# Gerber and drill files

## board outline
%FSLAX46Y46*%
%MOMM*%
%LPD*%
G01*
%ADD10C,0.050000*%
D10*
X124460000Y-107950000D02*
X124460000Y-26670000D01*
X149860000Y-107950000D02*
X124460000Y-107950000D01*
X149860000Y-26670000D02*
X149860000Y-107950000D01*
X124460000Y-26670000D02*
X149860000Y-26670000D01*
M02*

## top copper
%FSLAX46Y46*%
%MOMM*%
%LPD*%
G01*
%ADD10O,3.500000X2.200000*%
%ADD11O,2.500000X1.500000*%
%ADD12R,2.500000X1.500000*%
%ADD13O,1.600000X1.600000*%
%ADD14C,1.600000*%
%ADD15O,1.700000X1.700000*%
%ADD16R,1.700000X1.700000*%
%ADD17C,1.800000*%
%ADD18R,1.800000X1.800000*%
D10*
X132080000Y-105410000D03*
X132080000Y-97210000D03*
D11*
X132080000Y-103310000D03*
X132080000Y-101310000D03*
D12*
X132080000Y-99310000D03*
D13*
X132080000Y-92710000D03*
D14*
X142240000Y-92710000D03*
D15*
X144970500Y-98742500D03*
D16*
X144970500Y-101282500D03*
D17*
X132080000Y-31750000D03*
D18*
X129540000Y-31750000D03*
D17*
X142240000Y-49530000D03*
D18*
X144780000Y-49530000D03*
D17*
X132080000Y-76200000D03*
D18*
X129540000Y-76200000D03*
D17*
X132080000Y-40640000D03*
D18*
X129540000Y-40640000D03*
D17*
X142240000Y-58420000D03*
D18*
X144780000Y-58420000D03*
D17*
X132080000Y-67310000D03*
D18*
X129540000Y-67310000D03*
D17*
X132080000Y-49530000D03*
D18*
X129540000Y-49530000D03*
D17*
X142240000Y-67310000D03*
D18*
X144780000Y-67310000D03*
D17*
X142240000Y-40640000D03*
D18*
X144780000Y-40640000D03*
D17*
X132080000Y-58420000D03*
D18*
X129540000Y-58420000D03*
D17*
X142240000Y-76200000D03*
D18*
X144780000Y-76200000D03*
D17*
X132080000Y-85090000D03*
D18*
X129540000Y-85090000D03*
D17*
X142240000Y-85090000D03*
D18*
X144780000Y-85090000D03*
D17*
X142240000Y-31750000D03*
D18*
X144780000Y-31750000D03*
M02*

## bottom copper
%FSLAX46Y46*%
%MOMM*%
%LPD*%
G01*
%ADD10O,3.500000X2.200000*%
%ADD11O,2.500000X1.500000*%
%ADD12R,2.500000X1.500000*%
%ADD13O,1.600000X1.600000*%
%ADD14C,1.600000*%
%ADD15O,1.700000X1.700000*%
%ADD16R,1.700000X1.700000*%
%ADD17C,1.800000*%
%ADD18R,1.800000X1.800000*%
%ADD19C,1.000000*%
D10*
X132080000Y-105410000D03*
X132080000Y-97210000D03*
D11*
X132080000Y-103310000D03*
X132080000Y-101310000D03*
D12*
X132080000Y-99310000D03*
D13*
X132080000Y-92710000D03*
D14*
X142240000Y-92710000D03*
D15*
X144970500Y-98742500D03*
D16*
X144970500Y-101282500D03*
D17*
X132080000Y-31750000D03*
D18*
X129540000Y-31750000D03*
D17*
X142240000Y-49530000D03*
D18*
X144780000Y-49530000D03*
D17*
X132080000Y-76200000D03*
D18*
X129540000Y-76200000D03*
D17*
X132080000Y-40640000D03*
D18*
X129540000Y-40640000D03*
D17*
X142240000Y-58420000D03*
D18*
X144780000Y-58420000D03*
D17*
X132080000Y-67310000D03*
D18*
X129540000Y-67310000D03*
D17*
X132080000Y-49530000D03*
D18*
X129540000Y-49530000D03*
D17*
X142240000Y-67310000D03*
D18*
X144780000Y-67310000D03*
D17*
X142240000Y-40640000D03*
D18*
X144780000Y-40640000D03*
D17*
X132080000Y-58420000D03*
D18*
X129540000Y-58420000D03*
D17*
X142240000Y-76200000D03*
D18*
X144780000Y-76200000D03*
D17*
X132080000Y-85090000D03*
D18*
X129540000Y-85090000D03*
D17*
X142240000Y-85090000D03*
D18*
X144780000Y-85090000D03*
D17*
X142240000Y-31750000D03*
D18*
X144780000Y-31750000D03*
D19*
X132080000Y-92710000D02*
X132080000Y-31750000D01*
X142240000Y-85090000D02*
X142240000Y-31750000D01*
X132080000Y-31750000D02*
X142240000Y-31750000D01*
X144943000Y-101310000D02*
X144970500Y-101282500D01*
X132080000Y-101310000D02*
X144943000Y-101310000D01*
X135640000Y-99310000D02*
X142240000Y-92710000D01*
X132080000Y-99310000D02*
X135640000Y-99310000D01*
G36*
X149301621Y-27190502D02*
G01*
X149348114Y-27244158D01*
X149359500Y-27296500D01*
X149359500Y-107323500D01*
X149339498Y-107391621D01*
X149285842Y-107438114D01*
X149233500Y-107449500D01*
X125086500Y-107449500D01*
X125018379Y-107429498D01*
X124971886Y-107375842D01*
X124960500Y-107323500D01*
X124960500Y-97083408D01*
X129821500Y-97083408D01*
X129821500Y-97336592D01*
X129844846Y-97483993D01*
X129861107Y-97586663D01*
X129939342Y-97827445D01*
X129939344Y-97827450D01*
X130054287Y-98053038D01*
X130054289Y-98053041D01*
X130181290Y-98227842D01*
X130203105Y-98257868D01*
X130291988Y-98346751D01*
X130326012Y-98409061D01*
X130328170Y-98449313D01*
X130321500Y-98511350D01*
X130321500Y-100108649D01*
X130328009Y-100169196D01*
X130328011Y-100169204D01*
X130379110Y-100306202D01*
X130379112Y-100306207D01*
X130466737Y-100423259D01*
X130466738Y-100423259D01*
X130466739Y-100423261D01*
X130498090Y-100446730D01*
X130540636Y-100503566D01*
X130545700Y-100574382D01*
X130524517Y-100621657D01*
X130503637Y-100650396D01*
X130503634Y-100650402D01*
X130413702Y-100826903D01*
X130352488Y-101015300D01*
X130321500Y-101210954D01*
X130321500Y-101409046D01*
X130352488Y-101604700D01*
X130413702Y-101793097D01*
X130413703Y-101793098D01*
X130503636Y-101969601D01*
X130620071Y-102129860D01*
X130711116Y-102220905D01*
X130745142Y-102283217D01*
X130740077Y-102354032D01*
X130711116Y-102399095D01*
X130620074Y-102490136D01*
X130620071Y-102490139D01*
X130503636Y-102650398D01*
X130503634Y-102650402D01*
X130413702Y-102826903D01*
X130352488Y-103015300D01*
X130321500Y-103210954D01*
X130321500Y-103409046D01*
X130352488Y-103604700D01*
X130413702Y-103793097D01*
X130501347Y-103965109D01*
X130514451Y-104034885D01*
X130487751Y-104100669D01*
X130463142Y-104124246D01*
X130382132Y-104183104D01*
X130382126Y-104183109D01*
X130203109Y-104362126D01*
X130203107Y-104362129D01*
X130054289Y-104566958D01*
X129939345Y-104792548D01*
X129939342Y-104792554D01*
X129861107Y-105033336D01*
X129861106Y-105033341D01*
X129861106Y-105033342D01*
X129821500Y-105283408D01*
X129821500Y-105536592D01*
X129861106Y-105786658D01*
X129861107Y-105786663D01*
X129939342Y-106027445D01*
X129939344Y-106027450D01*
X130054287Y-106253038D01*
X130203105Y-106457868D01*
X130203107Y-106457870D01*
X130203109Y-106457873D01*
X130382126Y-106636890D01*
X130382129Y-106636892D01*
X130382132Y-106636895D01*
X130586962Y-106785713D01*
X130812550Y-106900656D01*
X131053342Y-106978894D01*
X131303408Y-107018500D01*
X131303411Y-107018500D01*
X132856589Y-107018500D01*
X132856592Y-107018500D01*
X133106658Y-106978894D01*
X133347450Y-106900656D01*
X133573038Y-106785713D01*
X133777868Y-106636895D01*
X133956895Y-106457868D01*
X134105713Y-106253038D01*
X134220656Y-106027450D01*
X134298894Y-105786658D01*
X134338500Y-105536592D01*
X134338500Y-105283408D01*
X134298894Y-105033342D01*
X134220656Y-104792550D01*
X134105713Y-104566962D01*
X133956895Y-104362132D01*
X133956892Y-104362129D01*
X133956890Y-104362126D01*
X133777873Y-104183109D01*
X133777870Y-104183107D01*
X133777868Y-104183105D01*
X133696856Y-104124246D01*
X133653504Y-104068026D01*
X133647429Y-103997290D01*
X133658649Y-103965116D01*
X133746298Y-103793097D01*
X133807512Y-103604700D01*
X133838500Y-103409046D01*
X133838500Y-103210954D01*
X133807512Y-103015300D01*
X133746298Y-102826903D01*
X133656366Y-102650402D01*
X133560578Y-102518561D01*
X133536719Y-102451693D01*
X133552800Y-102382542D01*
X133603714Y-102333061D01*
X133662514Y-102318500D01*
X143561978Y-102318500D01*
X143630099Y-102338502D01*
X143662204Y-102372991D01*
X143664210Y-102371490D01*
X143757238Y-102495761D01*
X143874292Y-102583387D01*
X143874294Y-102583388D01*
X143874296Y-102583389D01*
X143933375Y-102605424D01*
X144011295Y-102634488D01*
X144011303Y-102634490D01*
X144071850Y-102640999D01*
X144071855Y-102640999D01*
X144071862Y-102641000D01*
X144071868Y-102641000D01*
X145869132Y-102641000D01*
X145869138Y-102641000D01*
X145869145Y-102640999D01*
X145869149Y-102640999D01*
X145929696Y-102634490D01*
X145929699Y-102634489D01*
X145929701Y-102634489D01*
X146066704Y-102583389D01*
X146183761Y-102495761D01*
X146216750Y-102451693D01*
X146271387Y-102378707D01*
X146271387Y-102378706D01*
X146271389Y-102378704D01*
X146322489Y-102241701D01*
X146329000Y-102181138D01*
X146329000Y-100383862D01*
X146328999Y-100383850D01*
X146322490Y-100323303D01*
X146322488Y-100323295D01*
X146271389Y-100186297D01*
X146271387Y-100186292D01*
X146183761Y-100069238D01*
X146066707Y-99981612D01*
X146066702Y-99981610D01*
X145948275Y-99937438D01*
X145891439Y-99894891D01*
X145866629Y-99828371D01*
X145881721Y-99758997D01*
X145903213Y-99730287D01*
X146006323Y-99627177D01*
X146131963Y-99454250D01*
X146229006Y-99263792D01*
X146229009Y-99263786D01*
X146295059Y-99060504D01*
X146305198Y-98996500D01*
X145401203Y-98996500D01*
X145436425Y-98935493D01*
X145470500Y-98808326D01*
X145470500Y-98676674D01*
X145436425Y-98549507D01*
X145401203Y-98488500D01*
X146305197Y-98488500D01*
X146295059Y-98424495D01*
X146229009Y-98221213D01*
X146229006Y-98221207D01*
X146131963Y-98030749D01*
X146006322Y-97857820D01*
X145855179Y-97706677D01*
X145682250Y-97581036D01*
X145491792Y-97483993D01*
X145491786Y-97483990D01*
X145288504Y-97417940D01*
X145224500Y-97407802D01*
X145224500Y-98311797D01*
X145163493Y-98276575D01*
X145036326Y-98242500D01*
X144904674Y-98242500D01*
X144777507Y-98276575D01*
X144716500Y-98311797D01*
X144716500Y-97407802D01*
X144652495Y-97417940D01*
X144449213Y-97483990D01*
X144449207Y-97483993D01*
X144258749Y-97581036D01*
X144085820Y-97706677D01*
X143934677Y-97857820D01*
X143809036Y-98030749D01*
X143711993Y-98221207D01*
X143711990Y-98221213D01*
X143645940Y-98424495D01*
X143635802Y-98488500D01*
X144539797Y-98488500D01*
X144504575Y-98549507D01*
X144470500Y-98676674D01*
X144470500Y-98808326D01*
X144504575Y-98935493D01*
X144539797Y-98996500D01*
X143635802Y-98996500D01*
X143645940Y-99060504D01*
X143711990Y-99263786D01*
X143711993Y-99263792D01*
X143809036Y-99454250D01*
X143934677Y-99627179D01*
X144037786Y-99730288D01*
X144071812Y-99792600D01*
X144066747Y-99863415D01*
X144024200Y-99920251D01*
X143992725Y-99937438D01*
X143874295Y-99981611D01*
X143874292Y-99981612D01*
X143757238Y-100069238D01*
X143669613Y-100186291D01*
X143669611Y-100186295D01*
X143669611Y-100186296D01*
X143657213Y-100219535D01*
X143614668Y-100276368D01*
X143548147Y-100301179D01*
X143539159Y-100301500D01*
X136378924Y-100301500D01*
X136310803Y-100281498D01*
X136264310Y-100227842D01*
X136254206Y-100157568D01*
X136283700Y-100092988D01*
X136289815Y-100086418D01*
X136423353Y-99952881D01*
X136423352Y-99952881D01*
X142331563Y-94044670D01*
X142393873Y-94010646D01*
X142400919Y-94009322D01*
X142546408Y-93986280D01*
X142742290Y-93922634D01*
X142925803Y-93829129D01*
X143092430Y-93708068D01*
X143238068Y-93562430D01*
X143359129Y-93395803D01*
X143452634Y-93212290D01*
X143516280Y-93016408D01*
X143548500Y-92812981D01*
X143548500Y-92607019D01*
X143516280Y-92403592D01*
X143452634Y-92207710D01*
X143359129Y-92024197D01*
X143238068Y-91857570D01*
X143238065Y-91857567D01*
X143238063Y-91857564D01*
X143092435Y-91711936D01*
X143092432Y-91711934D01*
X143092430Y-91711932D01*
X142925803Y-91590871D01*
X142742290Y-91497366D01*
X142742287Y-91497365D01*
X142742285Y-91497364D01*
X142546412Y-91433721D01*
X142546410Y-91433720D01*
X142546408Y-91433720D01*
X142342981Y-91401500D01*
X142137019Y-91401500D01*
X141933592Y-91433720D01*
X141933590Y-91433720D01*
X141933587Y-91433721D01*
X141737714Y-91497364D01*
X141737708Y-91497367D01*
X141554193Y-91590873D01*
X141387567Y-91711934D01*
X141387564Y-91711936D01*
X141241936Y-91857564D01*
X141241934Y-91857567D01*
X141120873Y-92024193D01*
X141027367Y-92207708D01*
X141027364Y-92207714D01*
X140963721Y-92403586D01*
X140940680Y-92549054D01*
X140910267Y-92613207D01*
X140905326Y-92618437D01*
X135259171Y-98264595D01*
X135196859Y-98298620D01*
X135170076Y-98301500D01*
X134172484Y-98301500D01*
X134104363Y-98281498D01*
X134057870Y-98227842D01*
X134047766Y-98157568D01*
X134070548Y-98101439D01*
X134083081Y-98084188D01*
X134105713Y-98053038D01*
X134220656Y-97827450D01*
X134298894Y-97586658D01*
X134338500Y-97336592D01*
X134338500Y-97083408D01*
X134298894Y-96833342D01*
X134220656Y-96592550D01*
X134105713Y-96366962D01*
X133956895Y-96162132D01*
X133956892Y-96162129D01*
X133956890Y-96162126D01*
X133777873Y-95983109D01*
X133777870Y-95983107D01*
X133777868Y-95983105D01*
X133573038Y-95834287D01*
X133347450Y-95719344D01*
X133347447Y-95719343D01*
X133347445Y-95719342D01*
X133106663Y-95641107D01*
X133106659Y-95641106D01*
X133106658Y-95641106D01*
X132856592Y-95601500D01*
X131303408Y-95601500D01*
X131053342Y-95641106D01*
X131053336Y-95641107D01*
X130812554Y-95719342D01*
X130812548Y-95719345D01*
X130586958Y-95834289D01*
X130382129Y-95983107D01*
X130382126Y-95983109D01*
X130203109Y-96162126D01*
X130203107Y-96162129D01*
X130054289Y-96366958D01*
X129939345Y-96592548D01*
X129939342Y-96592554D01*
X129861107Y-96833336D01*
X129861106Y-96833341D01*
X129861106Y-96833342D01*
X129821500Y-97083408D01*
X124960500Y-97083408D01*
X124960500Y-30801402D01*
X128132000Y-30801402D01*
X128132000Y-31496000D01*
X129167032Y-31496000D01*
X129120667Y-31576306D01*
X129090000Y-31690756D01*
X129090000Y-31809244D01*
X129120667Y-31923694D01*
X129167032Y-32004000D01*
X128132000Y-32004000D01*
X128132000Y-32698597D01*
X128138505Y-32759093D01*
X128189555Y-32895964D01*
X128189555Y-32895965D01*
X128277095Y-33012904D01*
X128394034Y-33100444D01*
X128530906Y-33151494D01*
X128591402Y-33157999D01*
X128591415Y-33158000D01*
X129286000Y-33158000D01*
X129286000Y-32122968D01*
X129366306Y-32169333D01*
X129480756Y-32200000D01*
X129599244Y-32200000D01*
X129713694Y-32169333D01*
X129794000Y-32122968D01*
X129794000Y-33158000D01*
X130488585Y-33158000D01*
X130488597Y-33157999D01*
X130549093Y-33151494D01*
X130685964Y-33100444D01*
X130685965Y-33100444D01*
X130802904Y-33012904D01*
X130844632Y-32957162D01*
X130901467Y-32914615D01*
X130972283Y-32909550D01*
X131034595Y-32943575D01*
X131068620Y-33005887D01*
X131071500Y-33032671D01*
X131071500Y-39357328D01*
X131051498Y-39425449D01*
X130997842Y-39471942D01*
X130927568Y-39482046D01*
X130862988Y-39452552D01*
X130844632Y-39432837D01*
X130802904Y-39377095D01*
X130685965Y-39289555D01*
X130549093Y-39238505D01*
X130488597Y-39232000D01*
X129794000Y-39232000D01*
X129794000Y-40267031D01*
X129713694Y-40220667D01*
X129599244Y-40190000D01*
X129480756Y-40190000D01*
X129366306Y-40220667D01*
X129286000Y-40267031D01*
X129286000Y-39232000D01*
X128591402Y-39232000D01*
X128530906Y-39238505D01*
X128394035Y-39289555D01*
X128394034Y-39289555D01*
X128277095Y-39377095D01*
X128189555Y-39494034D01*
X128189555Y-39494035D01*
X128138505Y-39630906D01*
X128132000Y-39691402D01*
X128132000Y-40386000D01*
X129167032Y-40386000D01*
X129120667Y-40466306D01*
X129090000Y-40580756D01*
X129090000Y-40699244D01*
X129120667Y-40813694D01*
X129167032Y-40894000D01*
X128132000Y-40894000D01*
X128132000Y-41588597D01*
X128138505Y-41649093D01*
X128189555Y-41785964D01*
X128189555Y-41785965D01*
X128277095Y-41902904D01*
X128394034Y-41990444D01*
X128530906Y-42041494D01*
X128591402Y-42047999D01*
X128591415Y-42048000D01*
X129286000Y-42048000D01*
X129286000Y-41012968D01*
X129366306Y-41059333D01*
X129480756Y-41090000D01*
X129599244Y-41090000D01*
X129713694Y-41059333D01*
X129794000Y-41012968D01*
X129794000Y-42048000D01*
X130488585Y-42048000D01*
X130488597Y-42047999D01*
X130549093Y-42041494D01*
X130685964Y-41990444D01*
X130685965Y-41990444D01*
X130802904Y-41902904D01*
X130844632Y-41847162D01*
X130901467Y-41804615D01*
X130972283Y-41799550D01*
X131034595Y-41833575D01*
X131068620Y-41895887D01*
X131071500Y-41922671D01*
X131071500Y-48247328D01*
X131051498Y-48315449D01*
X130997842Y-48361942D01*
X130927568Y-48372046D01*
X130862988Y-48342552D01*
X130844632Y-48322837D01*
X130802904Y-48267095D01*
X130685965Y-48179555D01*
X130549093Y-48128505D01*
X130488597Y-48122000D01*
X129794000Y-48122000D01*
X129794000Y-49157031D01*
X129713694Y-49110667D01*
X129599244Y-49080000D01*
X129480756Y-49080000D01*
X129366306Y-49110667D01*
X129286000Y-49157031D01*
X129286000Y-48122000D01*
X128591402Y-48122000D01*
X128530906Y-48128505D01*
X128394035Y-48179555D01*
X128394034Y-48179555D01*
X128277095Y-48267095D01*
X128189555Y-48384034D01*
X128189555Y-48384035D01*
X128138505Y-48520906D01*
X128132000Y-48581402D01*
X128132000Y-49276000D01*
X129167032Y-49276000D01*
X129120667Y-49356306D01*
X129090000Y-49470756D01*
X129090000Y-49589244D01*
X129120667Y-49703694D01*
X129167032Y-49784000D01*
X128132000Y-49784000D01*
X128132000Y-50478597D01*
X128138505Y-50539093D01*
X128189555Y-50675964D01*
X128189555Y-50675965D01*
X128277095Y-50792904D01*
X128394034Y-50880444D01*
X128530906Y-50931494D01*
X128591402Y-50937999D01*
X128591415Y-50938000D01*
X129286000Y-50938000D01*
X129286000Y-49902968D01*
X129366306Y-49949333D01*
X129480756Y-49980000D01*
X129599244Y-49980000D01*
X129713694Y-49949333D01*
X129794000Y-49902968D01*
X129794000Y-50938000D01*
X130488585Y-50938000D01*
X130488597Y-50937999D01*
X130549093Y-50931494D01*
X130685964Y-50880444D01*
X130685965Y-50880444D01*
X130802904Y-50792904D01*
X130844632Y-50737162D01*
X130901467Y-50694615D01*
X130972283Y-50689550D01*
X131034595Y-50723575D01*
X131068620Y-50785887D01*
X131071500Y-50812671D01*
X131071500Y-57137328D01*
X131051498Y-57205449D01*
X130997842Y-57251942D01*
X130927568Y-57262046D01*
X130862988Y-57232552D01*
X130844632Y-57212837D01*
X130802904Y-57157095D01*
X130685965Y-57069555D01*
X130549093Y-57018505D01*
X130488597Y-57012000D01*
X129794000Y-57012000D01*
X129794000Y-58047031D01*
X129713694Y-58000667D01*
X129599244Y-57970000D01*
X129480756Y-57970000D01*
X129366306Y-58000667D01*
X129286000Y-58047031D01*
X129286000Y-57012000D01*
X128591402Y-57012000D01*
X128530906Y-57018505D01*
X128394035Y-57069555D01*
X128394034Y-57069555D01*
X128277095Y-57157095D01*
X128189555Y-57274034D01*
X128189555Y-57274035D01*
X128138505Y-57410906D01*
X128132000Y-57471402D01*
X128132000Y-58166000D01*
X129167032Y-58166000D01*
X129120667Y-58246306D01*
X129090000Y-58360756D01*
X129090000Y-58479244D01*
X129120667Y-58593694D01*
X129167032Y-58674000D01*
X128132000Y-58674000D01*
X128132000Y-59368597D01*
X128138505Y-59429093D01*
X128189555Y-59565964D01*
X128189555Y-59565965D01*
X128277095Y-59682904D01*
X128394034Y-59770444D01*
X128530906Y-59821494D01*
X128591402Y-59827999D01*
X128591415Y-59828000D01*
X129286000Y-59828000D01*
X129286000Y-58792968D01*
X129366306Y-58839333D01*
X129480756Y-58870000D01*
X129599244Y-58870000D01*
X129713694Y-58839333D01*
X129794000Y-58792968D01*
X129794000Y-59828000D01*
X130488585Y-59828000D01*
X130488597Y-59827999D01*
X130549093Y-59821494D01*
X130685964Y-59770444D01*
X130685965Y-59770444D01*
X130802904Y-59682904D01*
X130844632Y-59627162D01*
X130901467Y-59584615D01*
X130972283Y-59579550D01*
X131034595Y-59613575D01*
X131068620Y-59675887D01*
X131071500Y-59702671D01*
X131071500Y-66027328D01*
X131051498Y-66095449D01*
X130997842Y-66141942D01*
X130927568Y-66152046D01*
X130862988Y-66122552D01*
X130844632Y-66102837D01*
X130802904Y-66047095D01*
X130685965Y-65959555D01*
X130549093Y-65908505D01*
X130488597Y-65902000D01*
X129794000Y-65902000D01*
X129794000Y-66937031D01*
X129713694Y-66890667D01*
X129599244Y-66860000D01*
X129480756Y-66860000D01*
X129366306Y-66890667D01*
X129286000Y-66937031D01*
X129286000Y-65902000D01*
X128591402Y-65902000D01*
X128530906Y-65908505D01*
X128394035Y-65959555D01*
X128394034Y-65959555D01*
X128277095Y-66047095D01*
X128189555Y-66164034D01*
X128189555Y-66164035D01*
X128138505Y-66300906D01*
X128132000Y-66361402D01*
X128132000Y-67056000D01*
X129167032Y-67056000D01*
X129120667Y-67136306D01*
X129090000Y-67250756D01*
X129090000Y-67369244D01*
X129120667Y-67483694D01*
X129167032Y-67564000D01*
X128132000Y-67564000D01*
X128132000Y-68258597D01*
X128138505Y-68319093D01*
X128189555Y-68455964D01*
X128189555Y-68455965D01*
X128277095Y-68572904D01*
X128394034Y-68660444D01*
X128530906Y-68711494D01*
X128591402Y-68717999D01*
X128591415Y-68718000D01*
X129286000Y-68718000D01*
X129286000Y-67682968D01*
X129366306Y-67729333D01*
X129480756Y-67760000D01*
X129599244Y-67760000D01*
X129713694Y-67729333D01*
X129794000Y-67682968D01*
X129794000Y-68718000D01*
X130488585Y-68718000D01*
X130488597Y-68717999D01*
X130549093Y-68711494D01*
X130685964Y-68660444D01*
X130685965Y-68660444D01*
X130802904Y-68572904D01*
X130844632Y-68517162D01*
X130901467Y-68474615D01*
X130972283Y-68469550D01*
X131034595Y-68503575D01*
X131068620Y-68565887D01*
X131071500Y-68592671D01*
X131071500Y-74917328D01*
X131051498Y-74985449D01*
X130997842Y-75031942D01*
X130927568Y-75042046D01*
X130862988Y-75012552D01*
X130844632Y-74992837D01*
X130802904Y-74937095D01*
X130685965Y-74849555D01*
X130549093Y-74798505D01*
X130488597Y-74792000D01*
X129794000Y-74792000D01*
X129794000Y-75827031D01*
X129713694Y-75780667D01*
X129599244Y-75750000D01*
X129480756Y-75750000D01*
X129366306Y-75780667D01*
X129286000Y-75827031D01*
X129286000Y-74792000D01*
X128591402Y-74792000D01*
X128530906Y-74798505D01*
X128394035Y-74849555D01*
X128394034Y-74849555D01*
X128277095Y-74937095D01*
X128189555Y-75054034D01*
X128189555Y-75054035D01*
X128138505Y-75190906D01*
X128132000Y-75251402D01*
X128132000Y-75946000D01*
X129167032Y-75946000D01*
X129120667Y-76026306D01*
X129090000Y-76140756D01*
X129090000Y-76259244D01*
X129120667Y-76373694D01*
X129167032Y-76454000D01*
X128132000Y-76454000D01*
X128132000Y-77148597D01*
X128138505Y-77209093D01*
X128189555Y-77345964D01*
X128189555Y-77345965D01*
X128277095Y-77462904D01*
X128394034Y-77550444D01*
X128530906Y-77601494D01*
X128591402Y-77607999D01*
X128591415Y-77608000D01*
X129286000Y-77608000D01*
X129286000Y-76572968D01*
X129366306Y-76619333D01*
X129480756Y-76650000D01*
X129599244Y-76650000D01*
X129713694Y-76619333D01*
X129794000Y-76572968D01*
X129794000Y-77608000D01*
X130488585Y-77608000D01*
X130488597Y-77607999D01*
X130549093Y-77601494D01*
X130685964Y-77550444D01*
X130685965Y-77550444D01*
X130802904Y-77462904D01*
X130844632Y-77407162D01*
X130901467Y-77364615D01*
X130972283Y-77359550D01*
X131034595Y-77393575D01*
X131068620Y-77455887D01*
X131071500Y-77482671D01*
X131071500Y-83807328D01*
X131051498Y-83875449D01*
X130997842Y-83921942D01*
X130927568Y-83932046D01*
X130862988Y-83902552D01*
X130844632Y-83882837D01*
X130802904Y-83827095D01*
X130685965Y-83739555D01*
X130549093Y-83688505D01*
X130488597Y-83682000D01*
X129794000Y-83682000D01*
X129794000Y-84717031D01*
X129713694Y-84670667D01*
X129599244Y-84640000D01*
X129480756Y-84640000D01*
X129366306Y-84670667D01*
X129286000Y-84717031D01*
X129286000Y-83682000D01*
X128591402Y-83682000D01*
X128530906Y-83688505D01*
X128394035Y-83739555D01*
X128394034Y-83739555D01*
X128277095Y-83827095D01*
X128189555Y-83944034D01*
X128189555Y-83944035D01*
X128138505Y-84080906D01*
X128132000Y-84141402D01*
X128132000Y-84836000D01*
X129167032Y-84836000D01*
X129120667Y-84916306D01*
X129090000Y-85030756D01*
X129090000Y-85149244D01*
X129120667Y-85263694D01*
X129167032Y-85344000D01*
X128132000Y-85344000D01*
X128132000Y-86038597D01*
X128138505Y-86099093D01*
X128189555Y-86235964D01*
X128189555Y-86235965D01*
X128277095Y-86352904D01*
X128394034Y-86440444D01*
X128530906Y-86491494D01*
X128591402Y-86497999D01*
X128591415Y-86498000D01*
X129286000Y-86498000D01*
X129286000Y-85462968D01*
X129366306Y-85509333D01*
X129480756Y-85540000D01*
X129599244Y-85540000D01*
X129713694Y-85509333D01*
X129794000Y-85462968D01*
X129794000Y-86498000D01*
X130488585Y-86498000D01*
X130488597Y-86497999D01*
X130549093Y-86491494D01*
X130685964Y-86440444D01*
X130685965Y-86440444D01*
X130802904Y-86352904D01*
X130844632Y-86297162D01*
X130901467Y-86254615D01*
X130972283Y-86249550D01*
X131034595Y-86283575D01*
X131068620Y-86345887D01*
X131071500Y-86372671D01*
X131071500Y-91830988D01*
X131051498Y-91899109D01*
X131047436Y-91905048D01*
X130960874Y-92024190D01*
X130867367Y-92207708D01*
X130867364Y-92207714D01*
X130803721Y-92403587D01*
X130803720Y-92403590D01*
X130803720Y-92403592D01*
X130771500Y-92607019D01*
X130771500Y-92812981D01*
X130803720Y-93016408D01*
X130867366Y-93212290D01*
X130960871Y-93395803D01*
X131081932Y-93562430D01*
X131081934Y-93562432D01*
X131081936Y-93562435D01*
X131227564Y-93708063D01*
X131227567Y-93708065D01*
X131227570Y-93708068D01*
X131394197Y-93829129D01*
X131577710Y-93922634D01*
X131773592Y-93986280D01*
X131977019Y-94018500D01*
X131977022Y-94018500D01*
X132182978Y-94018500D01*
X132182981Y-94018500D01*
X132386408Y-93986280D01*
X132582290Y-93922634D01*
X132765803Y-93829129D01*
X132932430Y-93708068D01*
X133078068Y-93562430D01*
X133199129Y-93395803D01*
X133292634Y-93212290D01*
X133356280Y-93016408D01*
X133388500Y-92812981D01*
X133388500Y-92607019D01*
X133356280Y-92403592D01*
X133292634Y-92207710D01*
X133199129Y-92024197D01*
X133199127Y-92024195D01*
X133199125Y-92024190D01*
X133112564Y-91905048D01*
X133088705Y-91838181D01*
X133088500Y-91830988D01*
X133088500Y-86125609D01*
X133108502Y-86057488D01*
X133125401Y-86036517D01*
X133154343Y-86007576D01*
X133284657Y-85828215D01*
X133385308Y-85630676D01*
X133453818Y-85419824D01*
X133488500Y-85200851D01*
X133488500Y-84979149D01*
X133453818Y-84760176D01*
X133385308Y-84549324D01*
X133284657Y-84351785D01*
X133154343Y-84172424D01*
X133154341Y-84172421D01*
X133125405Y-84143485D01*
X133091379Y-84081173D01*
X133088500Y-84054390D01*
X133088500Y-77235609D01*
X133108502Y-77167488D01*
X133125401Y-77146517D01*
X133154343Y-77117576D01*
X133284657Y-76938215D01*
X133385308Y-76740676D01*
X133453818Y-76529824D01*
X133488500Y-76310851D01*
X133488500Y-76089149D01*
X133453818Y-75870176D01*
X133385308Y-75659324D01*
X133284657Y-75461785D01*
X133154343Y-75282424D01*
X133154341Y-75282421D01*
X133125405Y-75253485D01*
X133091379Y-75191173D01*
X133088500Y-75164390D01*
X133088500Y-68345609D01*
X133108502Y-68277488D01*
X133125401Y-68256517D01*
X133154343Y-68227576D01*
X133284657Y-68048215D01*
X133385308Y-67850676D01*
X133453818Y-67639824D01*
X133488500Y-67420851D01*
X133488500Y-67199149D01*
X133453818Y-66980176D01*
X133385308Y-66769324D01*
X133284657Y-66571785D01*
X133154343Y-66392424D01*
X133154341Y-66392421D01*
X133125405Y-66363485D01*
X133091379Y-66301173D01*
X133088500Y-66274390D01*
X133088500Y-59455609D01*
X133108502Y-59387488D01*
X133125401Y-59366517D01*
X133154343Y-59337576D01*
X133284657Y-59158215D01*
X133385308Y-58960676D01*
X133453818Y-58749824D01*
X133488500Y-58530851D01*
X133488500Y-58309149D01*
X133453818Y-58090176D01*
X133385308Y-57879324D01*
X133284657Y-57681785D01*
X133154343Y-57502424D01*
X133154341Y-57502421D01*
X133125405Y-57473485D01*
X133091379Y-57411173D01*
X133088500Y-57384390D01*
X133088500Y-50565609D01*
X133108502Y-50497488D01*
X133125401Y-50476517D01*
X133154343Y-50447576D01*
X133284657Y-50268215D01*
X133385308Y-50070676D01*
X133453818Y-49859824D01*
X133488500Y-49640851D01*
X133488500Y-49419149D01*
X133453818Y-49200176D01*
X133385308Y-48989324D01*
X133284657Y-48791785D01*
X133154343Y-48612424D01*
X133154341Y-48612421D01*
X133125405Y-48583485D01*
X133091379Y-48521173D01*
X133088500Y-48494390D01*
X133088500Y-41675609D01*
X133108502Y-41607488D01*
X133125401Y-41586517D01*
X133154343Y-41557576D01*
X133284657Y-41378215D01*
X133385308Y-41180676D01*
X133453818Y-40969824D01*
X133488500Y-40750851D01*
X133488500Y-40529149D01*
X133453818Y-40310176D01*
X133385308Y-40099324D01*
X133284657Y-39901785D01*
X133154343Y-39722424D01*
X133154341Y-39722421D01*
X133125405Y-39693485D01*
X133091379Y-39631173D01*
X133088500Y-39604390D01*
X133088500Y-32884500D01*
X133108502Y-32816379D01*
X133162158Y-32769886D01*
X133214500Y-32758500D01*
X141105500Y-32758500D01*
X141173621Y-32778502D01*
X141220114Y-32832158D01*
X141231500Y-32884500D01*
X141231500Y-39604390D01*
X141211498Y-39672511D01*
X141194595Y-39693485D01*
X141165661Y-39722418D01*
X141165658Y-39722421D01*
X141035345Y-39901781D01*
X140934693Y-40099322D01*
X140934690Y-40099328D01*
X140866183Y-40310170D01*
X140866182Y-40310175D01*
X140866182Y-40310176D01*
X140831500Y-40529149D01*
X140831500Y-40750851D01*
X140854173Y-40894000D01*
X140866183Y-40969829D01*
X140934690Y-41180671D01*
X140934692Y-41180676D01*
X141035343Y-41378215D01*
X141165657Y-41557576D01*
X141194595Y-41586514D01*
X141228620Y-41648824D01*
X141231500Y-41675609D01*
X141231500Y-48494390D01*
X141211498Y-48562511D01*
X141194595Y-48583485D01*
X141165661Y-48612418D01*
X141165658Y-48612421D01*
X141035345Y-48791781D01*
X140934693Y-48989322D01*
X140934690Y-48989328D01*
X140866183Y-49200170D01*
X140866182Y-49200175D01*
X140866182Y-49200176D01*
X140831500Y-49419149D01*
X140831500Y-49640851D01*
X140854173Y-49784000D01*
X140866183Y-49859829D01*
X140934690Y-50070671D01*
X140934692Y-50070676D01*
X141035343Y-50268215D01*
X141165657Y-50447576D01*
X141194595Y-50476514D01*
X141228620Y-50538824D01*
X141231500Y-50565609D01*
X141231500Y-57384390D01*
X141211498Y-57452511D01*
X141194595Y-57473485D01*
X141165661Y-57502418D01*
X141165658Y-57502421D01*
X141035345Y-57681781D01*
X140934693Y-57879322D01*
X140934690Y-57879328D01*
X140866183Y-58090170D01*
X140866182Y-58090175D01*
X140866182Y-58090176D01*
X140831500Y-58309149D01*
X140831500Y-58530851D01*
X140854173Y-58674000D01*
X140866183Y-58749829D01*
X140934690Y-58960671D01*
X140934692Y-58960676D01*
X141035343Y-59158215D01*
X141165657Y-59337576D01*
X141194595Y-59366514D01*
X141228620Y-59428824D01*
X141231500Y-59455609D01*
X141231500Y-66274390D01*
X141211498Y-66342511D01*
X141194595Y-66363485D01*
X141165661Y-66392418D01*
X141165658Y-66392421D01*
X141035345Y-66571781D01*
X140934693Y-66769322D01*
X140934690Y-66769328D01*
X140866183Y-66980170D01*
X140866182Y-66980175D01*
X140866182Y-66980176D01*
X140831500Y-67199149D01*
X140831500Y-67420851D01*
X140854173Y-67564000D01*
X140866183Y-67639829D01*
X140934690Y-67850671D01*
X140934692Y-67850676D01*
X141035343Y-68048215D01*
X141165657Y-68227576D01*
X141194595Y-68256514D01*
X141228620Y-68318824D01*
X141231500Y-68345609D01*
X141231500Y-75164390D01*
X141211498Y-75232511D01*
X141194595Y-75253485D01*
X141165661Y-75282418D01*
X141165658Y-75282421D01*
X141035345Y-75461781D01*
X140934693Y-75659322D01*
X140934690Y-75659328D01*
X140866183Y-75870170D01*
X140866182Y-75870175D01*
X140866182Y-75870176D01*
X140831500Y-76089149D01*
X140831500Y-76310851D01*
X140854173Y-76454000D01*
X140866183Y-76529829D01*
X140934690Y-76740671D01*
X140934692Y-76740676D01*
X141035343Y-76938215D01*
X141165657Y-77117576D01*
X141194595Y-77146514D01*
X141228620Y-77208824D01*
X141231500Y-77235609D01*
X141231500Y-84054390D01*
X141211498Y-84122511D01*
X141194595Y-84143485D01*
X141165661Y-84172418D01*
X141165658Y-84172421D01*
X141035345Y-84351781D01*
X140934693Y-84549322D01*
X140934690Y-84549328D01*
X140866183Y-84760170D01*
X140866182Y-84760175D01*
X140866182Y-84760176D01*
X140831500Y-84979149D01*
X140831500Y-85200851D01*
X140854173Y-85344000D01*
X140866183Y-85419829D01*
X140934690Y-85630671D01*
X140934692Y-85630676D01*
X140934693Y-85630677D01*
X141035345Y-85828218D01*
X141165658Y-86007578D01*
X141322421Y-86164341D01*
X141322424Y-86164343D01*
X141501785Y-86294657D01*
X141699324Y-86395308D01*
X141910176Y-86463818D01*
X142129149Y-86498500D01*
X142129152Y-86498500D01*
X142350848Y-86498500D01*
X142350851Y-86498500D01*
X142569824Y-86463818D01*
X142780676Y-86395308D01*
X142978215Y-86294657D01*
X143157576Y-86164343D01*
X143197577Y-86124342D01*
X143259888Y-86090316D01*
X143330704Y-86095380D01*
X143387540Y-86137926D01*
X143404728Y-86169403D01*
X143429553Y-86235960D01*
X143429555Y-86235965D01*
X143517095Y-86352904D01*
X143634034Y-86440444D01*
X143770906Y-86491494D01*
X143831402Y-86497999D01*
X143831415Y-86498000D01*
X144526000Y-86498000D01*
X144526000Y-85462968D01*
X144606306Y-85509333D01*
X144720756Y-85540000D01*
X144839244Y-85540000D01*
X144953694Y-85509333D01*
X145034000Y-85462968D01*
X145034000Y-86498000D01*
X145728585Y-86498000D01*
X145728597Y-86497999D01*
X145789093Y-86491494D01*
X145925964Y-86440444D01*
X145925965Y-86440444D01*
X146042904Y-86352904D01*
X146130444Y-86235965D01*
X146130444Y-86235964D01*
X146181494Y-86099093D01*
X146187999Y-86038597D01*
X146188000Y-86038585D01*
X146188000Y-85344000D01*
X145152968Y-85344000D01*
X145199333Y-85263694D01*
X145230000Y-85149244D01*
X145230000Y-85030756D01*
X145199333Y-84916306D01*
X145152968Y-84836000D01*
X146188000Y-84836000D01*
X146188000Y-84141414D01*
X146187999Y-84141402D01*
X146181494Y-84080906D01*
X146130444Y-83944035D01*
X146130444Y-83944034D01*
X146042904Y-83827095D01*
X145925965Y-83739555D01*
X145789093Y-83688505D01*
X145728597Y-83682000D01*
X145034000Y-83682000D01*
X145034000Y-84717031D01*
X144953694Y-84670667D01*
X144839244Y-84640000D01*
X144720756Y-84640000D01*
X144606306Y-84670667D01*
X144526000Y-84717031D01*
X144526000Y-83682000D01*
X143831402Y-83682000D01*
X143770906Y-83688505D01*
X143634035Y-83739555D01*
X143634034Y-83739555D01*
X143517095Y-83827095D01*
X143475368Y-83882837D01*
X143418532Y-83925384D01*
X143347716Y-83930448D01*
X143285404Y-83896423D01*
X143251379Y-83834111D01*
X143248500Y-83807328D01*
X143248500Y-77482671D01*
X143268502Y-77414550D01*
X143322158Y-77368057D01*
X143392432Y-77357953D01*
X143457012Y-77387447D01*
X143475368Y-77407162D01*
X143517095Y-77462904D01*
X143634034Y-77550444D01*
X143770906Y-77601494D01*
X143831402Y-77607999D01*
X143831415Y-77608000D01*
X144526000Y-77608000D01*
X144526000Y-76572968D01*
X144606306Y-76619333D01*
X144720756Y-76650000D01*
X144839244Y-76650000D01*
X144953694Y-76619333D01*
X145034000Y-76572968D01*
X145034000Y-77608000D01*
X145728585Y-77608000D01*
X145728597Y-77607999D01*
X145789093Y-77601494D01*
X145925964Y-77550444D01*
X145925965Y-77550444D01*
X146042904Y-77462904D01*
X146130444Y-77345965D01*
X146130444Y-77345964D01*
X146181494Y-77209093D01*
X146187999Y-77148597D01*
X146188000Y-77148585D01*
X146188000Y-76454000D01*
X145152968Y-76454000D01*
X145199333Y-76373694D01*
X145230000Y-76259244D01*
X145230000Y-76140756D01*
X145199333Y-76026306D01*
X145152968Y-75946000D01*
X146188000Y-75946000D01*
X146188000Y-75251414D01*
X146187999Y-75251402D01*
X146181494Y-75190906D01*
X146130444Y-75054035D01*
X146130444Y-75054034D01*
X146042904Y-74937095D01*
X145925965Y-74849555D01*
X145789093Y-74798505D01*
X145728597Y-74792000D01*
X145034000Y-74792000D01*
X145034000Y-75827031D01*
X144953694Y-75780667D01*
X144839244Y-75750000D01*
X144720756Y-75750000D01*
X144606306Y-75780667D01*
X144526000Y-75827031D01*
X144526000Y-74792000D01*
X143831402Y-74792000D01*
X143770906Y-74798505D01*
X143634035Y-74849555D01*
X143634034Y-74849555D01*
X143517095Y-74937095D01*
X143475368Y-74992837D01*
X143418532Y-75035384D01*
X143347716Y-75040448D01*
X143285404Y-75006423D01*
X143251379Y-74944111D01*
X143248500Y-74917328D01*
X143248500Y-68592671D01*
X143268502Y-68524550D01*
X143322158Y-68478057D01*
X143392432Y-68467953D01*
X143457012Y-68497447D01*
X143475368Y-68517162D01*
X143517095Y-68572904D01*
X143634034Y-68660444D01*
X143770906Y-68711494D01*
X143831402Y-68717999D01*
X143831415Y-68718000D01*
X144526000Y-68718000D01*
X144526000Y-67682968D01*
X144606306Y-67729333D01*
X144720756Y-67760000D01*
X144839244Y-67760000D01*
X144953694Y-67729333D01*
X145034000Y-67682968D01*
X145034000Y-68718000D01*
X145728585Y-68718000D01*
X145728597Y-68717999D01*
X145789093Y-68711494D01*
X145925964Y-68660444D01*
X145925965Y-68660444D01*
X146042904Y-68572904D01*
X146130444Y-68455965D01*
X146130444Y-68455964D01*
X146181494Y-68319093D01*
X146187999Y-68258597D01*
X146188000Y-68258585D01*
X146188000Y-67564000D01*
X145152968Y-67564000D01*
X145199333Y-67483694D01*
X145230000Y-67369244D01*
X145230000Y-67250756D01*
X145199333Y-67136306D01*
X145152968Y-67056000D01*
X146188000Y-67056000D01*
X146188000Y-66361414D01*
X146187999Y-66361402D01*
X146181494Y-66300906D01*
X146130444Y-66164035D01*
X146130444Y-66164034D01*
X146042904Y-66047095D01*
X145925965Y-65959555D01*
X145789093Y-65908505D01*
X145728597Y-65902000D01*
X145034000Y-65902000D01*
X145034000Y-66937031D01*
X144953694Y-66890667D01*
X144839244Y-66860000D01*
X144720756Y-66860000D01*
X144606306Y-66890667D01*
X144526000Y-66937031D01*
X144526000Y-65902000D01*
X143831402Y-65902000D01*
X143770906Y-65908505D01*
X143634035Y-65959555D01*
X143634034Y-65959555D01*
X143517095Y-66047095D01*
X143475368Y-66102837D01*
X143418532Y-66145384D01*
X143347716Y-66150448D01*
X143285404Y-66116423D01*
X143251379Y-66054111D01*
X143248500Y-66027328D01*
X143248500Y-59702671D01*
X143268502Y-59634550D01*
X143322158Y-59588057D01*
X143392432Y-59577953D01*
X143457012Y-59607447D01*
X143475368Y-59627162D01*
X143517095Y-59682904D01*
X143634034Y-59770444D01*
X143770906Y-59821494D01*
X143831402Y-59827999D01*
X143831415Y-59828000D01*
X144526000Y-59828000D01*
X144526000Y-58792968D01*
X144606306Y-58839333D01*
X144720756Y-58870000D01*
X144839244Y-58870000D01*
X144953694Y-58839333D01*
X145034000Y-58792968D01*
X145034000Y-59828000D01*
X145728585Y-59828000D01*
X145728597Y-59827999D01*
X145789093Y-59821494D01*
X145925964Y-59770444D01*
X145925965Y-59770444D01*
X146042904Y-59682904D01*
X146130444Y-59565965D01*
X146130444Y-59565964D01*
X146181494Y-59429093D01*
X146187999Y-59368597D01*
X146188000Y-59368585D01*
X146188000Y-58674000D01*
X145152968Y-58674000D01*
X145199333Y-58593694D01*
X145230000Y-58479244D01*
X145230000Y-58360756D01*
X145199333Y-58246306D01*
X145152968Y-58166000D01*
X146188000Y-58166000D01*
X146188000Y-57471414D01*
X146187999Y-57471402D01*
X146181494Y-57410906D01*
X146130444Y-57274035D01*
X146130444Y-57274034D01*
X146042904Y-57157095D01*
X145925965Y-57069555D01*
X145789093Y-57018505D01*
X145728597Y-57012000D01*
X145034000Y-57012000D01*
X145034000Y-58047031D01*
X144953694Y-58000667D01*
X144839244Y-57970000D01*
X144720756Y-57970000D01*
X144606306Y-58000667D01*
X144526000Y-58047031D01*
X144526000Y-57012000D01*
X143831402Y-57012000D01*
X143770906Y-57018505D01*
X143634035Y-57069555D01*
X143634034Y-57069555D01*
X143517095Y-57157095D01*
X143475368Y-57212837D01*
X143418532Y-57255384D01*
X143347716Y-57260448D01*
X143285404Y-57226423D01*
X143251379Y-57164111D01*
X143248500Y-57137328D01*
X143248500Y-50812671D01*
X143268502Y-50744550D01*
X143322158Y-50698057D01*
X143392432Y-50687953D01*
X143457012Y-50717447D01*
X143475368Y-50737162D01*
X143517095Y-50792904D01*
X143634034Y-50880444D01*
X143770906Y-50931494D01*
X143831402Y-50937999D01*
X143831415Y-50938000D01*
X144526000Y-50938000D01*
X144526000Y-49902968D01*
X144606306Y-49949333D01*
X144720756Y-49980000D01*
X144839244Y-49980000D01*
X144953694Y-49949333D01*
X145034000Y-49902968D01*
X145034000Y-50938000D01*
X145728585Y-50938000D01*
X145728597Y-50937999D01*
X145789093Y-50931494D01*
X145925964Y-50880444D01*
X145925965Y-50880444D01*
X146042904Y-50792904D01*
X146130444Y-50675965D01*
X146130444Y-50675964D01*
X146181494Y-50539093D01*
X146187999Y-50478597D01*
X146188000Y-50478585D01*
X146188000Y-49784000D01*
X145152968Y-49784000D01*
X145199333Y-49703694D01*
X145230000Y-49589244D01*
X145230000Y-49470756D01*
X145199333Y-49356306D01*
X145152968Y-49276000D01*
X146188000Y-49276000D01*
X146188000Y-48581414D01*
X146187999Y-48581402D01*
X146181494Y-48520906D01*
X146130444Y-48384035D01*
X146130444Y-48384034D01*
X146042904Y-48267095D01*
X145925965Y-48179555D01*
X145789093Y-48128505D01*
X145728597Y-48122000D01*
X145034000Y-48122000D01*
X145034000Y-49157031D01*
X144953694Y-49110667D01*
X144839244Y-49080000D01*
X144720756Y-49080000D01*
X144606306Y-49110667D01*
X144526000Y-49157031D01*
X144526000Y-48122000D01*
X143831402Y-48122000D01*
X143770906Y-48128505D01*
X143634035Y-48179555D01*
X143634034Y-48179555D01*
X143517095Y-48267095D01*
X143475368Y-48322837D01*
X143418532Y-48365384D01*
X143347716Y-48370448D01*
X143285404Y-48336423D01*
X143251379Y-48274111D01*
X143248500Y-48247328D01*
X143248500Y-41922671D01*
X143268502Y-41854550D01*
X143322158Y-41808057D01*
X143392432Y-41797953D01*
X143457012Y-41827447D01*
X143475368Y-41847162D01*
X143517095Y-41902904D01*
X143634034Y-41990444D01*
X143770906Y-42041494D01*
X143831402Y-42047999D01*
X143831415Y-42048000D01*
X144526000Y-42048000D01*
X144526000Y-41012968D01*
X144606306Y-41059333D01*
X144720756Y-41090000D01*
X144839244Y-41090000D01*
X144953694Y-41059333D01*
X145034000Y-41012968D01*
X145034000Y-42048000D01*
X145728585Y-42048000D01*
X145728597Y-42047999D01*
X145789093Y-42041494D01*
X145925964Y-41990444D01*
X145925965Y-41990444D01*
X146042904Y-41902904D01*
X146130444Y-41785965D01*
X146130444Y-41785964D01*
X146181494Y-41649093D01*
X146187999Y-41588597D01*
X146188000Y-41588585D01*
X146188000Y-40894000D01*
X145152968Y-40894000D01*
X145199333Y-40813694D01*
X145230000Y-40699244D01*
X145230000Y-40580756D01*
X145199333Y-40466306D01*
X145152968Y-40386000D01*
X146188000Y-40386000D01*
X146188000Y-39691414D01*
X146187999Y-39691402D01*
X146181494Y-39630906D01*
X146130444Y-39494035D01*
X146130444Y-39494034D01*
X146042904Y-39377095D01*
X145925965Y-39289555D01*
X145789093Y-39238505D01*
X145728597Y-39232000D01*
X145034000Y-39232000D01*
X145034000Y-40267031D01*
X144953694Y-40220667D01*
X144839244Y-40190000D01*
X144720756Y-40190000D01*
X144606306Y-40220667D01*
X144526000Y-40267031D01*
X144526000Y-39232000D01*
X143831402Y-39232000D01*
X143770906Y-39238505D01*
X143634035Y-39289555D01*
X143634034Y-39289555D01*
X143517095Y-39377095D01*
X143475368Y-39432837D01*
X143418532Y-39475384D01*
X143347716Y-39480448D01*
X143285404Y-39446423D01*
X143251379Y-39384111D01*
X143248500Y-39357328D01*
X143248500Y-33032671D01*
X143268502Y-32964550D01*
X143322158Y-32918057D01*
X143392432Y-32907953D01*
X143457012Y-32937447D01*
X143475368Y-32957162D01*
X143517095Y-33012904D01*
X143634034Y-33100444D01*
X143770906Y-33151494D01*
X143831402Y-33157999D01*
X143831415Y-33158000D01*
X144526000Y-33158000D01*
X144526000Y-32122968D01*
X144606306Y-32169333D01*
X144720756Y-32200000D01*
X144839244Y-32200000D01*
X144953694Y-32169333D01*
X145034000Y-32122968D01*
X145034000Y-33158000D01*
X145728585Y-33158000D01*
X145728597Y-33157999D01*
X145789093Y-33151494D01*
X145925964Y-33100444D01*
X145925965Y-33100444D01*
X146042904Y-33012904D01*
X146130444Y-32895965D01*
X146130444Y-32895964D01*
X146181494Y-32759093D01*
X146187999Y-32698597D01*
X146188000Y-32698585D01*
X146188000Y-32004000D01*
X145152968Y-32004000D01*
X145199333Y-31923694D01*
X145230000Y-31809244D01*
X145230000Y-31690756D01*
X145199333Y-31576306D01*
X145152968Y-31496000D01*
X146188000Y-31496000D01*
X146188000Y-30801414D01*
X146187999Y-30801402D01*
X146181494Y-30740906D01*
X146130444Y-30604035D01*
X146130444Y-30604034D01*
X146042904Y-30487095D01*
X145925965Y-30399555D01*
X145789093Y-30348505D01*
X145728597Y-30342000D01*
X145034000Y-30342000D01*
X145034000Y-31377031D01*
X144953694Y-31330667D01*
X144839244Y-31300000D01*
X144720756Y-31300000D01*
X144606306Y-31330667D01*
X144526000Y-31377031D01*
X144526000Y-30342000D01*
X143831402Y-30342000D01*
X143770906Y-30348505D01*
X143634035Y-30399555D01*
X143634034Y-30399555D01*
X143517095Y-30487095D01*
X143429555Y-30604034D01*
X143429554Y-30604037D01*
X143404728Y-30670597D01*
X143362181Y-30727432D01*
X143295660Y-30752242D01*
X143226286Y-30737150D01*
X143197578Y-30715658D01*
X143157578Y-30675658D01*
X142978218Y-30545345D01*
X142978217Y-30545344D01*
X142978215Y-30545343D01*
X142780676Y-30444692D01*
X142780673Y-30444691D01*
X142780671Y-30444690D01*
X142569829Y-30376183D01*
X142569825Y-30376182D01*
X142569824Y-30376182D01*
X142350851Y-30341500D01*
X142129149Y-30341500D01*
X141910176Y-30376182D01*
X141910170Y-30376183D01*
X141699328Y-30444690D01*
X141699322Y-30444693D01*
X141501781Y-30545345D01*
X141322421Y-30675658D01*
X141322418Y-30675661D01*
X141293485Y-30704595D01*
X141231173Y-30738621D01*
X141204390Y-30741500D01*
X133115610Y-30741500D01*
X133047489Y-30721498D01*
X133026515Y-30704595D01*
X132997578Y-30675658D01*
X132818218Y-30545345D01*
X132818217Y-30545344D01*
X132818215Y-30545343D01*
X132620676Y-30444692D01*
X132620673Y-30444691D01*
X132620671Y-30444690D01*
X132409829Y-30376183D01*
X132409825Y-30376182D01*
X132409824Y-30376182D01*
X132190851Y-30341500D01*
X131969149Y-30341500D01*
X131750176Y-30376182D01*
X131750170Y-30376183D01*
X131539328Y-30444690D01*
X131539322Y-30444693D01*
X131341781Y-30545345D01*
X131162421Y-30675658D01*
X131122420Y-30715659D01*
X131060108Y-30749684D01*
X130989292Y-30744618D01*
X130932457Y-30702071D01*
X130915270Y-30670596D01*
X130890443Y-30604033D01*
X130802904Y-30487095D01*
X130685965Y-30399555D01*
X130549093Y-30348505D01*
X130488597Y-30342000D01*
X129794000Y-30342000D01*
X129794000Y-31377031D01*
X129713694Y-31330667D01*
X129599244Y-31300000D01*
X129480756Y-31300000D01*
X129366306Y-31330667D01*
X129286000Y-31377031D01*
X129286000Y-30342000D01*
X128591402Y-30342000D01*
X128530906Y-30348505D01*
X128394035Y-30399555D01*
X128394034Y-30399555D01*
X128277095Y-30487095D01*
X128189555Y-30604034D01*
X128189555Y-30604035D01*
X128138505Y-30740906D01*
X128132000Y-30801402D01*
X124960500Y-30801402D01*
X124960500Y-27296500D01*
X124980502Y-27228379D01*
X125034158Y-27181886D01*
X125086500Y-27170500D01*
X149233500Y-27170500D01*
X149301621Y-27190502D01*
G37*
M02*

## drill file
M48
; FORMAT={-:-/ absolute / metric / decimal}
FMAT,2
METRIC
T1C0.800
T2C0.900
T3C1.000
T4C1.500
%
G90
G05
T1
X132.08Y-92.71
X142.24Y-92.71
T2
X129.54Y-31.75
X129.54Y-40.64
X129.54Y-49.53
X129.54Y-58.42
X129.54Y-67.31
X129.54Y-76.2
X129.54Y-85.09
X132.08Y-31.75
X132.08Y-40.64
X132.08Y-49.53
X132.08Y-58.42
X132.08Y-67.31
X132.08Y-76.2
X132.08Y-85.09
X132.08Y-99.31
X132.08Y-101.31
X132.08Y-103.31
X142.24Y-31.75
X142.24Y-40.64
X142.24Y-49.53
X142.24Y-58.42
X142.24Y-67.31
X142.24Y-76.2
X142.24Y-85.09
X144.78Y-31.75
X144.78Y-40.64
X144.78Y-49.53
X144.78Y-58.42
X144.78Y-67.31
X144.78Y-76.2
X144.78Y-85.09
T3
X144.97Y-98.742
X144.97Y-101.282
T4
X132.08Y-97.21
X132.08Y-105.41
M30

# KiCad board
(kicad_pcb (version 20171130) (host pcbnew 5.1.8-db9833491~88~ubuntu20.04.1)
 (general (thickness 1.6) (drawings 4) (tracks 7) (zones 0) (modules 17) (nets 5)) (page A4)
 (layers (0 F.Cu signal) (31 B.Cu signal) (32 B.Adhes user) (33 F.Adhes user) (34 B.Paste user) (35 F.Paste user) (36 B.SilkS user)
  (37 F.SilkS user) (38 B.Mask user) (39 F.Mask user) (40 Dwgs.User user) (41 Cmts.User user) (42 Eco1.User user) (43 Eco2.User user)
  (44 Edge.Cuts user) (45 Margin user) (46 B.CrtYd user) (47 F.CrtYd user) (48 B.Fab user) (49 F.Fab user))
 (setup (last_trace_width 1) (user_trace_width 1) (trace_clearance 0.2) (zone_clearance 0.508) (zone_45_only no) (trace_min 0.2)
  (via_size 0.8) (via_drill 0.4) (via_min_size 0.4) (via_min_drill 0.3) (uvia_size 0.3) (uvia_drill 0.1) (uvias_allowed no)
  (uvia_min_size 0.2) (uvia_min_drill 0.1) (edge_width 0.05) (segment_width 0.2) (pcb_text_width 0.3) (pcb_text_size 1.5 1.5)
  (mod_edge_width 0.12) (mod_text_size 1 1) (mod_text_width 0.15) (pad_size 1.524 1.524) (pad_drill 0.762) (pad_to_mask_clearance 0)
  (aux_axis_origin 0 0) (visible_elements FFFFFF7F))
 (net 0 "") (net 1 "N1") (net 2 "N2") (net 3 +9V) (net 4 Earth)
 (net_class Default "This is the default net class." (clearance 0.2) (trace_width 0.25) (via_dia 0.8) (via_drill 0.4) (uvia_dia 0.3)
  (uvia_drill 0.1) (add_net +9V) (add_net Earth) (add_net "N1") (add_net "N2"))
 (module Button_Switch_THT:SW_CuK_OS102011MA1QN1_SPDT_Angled (layer F.Cu) (at 132.08 99.31 270)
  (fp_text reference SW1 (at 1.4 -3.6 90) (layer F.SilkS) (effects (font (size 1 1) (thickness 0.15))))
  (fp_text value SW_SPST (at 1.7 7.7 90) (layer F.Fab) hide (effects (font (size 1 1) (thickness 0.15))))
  (pad "" thru_hole oval (at 6.1 0 270) (size 2.2 3.5) (drill 1.5) (layers *.Cu *.Mask))
  (pad "" thru_hole oval (at -2.1 0 270) (size 2.2 3.5) (drill 1.5) (layers *.Cu *.Mask))
  (pad 3 thru_hole oval (at 4 0 270) (size 1.5 2.5) (drill 0.9) (layers *.Cu *.Mask))
  (pad 2 thru_hole oval (at 2 0 270) (size 1.5 2.5) (drill 0.9) (layers *.Cu *.Mask) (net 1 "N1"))
  (pad 1 thru_hole rect (at 0 0 270) (size 1.5 2.5) (drill 0.9) (layers *.Cu *.Mask) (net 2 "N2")))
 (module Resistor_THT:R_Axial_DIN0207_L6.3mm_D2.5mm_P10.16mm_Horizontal (layer F.Cu) (at 142.24 92.71 180)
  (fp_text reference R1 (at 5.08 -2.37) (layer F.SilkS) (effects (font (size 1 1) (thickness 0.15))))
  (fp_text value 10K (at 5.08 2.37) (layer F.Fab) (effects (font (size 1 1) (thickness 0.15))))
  (pad 2 thru_hole oval (at 10.16 0 180) (size 1.6 1.6) (drill 0.8) (layers *.Cu *.Mask) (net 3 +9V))
  (pad 1 thru_hole circle (at 0 0 180) (size 1.6 1.6) (drill 0.8) (layers *.Cu *.Mask) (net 2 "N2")))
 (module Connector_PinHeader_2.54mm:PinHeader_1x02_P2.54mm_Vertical (layer F.Cu) (at 144.9705 101.2825 180)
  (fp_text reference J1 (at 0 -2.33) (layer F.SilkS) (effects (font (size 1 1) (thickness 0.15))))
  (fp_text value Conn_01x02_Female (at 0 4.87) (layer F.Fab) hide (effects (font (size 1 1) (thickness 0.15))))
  (pad 2 thru_hole oval (at 0 2.54 180) (size 1.7 1.7) (drill 1) (layers *.Cu *.Mask) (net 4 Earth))
  (pad 1 thru_hole rect (at 0 0 180) (size 1.7 1.7) (drill 1) (layers *.Cu *.Mask) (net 1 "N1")))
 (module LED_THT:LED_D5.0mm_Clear (layer F.Cu) (at 129.54 31.75)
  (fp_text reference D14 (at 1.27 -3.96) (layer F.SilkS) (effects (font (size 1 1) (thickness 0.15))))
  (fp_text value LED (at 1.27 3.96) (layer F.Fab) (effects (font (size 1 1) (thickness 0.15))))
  (pad 2 thru_hole circle (at 2.54 0) (size 1.8 1.8) (drill 0.9) (layers *.Cu *.Mask) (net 3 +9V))
  (pad 1 thru_hole rect (at 0 0) (size 1.8 1.8) (drill 0.9) (layers *.Cu *.Mask) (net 4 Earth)))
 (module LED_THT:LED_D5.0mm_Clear (layer F.Cu) (at 144.78 49.53 180)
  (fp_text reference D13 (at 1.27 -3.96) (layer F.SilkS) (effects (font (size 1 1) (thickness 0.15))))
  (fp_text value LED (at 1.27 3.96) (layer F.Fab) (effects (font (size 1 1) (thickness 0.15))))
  (pad 2 thru_hole circle (at 2.54 0 180) (size 1.8 1.8) (drill 0.9) (layers *.Cu *.Mask) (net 3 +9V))
  (pad 1 thru_hole rect (at 0 0 180) (size 1.8 1.8) (drill 0.9) (layers *.Cu *.Mask) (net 4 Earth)))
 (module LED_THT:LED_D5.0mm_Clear (layer F.Cu) (at 129.54 76.2)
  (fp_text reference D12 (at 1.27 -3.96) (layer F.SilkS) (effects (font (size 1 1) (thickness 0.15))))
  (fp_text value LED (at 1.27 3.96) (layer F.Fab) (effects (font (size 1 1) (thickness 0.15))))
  (pad 2 thru_hole circle (at 2.54 0) (size 1.8 1.8) (drill 0.9) (layers *.Cu *.Mask) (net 3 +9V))
  (pad 1 thru_hole rect (at 0 0) (size 1.8 1.8) (drill 0.9) (layers *.Cu *.Mask) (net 4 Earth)))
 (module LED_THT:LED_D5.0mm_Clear (layer F.Cu) (at 129.54 40.64)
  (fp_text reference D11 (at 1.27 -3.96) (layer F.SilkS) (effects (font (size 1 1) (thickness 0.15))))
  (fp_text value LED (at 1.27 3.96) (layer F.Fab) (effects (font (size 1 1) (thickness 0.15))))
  (pad 2 thru_hole circle (at 2.54 0) (size 1.8 1.8) (drill 0.9) (layers *.Cu *.Mask) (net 3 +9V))
  (pad 1 thru_hole rect (at 0 0) (size 1.8 1.8) (drill 0.9) (layers *.Cu *.Mask) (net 4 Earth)))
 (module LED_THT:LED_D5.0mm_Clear (layer F.Cu) (at 144.78 58.42 180)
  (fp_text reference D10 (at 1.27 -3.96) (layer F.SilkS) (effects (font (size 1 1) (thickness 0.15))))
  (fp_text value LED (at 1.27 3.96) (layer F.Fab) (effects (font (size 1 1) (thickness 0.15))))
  (pad 2 thru_hole circle (at 2.54 0 180) (size 1.8 1.8) (drill 0.9) (layers *.Cu *.Mask) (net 3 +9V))
  (pad 1 thru_hole rect (at 0 0 180) (size 1.8 1.8) (drill 0.9) (layers *.Cu *.Mask) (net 4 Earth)))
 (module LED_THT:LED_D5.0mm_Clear (layer F.Cu) (at 129.54 67.31)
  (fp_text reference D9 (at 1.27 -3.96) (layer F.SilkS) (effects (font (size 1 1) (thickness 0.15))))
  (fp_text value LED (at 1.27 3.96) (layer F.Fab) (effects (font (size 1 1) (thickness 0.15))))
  (pad 2 thru_hole circle (at 2.54 0) (size 1.8 1.8) (drill 0.9) (layers *.Cu *.Mask) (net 3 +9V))
  (pad 1 thru_hole rect (at 0 0) (size 1.8 1.8) (drill 0.9) (layers *.Cu *.Mask) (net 4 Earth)))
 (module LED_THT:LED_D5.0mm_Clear (layer F.Cu) (at 129.54 49.53)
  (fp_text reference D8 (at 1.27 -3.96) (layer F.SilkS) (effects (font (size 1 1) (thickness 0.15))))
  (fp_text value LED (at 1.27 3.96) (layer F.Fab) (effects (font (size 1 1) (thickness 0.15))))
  (pad 2 thru_hole circle (at 2.54 0) (size 1.8 1.8) (drill 0.9) (layers *.Cu *.Mask) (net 3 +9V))
  (pad 1 thru_hole rect (at 0 0) (size 1.8 1.8) (drill 0.9) (layers *.Cu *.Mask) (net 4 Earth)))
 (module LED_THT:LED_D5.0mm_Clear (layer F.Cu) (at 144.78 67.31 180)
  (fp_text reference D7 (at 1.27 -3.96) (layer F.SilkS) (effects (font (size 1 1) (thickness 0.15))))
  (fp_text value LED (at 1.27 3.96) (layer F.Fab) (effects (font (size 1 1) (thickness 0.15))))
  (pad 2 thru_hole circle (at 2.54 0 180) (size 1.8 1.8) (drill 0.9) (layers *.Cu *.Mask) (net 3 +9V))
  (pad 1 thru_hole rect (at 0 0 180) (size 1.8 1.8) (drill 0.9) (layers *.Cu *.Mask) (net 4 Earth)))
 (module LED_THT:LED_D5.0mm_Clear (layer F.Cu) (at 144.78 40.64 180)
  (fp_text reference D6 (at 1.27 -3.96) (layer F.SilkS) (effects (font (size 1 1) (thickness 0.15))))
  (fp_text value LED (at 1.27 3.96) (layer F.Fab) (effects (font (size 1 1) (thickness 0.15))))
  (pad 2 thru_hole circle (at 2.54 0 180) (size 1.8 1.8) (drill 0.9) (layers *.Cu *.Mask) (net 3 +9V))
  (pad 1 thru_hole rect (at 0 0 180) (size 1.8 1.8) (drill 0.9) (layers *.Cu *.Mask) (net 4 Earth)))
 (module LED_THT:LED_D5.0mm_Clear (layer F.Cu) (at 129.54 58.42)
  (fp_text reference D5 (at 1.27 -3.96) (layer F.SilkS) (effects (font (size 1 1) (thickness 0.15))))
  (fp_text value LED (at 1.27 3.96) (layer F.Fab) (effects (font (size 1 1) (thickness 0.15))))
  (pad 2 thru_hole circle (at 2.54 0) (size 1.8 1.8) (drill 0.9) (layers *.Cu *.Mask) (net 3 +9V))
  (pad 1 thru_hole rect (at 0 0) (size 1.8 1.8) (drill 0.9) (layers *.Cu *.Mask) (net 4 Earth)))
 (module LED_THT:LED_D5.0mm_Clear (layer F.Cu) (at 144.78 76.2 180)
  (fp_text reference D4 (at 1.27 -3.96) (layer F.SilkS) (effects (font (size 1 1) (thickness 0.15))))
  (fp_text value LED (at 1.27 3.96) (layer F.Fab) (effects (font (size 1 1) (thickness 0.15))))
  (pad 2 thru_hole circle (at 2.54 0 180) (size 1.8 1.8) (drill 0.9) (layers *.Cu *.Mask) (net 3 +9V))
  (pad 1 thru_hole rect (at 0 0 180) (size 1.8 1.8) (drill 0.9) (layers *.Cu *.Mask) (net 4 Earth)))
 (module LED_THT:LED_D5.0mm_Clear (layer F.Cu) (at 129.54 85.09)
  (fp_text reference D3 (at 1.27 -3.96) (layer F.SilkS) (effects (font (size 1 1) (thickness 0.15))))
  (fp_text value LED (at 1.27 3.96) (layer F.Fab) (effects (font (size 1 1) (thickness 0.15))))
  (pad 2 thru_hole circle (at 2.54 0) (size 1.8 1.8) (drill 0.9) (layers *.Cu *.Mask) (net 3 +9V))
  (pad 1 thru_hole rect (at 0 0) (size 1.8 1.8) (drill 0.9) (layers *.Cu *.Mask) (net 4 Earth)))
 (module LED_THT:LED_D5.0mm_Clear (layer F.Cu) (at 144.78 85.09 180)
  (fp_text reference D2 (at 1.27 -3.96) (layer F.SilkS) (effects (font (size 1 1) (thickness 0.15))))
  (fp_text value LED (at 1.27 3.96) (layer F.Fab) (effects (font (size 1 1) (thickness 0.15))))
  (pad 2 thru_hole circle (at 2.54 0 180) (size 1.8 1.8) (drill 0.9) (layers *.Cu *.Mask) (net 3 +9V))
  (pad 1 thru_hole rect (at 0 0 180) (size 1.8 1.8) (drill 0.9) (layers *.Cu *.Mask) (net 4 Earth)))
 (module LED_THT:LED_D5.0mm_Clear (layer F.Cu) (at 144.78 31.75 180)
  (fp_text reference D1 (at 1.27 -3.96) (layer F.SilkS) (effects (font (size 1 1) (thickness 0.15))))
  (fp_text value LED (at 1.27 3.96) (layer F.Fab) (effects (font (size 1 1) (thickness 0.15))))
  (pad 2 thru_hole circle (at 2.54 0 180) (size 1.8 1.8) (drill 0.9) (layers *.Cu *.Mask) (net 3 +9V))
  (pad 1 thru_hole rect (at 0 0 180) (size 1.8 1.8) (drill 0.9) (layers *.Cu *.Mask) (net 4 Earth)))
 (gr_line (start 124.46 107.95) (end 124.46 26.67) (layer Edge.Cuts) (width 0.05))
 (gr_line (start 149.86 107.95) (end 124.46 107.95) (layer Edge.Cuts) (width 0.05))
 (gr_line (start 149.86 26.67) (end 149.86 107.95) (layer Edge.Cuts) (width 0.05))
 (gr_line (start 124.46 26.67) (end 149.86 26.67) (layer Edge.Cuts) (width 0.05))
 (segment (start 132.08 92.71) (end 132.08 31.75) (width 1) (layer B.Cu) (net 3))
 (segment (start 142.24 85.09) (end 142.24 31.75) (width 1) (layer B.Cu) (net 3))
 (segment (start 132.08 31.75) (end 142.24 31.75) (width 1) (layer B.Cu) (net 3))
 (segment (start 144.943 101.31) (end 144.9705 101.2825) (width 1) (layer B.Cu) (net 1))
 (segment (start 132.08 101.31) (end 144.943 101.31) (width 1) (layer B.Cu) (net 1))
 (segment (start 135.64 99.31) (end 142.24 92.71) (width 1) (layer B.Cu) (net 2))
 (segment (start 132.08 99.31) (end 135.64 99.31) (width 1) (layer B.Cu) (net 2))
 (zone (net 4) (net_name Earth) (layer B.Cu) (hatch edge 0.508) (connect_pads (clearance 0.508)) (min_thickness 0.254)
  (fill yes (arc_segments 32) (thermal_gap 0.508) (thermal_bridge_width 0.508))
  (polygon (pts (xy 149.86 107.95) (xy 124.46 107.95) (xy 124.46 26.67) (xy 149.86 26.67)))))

